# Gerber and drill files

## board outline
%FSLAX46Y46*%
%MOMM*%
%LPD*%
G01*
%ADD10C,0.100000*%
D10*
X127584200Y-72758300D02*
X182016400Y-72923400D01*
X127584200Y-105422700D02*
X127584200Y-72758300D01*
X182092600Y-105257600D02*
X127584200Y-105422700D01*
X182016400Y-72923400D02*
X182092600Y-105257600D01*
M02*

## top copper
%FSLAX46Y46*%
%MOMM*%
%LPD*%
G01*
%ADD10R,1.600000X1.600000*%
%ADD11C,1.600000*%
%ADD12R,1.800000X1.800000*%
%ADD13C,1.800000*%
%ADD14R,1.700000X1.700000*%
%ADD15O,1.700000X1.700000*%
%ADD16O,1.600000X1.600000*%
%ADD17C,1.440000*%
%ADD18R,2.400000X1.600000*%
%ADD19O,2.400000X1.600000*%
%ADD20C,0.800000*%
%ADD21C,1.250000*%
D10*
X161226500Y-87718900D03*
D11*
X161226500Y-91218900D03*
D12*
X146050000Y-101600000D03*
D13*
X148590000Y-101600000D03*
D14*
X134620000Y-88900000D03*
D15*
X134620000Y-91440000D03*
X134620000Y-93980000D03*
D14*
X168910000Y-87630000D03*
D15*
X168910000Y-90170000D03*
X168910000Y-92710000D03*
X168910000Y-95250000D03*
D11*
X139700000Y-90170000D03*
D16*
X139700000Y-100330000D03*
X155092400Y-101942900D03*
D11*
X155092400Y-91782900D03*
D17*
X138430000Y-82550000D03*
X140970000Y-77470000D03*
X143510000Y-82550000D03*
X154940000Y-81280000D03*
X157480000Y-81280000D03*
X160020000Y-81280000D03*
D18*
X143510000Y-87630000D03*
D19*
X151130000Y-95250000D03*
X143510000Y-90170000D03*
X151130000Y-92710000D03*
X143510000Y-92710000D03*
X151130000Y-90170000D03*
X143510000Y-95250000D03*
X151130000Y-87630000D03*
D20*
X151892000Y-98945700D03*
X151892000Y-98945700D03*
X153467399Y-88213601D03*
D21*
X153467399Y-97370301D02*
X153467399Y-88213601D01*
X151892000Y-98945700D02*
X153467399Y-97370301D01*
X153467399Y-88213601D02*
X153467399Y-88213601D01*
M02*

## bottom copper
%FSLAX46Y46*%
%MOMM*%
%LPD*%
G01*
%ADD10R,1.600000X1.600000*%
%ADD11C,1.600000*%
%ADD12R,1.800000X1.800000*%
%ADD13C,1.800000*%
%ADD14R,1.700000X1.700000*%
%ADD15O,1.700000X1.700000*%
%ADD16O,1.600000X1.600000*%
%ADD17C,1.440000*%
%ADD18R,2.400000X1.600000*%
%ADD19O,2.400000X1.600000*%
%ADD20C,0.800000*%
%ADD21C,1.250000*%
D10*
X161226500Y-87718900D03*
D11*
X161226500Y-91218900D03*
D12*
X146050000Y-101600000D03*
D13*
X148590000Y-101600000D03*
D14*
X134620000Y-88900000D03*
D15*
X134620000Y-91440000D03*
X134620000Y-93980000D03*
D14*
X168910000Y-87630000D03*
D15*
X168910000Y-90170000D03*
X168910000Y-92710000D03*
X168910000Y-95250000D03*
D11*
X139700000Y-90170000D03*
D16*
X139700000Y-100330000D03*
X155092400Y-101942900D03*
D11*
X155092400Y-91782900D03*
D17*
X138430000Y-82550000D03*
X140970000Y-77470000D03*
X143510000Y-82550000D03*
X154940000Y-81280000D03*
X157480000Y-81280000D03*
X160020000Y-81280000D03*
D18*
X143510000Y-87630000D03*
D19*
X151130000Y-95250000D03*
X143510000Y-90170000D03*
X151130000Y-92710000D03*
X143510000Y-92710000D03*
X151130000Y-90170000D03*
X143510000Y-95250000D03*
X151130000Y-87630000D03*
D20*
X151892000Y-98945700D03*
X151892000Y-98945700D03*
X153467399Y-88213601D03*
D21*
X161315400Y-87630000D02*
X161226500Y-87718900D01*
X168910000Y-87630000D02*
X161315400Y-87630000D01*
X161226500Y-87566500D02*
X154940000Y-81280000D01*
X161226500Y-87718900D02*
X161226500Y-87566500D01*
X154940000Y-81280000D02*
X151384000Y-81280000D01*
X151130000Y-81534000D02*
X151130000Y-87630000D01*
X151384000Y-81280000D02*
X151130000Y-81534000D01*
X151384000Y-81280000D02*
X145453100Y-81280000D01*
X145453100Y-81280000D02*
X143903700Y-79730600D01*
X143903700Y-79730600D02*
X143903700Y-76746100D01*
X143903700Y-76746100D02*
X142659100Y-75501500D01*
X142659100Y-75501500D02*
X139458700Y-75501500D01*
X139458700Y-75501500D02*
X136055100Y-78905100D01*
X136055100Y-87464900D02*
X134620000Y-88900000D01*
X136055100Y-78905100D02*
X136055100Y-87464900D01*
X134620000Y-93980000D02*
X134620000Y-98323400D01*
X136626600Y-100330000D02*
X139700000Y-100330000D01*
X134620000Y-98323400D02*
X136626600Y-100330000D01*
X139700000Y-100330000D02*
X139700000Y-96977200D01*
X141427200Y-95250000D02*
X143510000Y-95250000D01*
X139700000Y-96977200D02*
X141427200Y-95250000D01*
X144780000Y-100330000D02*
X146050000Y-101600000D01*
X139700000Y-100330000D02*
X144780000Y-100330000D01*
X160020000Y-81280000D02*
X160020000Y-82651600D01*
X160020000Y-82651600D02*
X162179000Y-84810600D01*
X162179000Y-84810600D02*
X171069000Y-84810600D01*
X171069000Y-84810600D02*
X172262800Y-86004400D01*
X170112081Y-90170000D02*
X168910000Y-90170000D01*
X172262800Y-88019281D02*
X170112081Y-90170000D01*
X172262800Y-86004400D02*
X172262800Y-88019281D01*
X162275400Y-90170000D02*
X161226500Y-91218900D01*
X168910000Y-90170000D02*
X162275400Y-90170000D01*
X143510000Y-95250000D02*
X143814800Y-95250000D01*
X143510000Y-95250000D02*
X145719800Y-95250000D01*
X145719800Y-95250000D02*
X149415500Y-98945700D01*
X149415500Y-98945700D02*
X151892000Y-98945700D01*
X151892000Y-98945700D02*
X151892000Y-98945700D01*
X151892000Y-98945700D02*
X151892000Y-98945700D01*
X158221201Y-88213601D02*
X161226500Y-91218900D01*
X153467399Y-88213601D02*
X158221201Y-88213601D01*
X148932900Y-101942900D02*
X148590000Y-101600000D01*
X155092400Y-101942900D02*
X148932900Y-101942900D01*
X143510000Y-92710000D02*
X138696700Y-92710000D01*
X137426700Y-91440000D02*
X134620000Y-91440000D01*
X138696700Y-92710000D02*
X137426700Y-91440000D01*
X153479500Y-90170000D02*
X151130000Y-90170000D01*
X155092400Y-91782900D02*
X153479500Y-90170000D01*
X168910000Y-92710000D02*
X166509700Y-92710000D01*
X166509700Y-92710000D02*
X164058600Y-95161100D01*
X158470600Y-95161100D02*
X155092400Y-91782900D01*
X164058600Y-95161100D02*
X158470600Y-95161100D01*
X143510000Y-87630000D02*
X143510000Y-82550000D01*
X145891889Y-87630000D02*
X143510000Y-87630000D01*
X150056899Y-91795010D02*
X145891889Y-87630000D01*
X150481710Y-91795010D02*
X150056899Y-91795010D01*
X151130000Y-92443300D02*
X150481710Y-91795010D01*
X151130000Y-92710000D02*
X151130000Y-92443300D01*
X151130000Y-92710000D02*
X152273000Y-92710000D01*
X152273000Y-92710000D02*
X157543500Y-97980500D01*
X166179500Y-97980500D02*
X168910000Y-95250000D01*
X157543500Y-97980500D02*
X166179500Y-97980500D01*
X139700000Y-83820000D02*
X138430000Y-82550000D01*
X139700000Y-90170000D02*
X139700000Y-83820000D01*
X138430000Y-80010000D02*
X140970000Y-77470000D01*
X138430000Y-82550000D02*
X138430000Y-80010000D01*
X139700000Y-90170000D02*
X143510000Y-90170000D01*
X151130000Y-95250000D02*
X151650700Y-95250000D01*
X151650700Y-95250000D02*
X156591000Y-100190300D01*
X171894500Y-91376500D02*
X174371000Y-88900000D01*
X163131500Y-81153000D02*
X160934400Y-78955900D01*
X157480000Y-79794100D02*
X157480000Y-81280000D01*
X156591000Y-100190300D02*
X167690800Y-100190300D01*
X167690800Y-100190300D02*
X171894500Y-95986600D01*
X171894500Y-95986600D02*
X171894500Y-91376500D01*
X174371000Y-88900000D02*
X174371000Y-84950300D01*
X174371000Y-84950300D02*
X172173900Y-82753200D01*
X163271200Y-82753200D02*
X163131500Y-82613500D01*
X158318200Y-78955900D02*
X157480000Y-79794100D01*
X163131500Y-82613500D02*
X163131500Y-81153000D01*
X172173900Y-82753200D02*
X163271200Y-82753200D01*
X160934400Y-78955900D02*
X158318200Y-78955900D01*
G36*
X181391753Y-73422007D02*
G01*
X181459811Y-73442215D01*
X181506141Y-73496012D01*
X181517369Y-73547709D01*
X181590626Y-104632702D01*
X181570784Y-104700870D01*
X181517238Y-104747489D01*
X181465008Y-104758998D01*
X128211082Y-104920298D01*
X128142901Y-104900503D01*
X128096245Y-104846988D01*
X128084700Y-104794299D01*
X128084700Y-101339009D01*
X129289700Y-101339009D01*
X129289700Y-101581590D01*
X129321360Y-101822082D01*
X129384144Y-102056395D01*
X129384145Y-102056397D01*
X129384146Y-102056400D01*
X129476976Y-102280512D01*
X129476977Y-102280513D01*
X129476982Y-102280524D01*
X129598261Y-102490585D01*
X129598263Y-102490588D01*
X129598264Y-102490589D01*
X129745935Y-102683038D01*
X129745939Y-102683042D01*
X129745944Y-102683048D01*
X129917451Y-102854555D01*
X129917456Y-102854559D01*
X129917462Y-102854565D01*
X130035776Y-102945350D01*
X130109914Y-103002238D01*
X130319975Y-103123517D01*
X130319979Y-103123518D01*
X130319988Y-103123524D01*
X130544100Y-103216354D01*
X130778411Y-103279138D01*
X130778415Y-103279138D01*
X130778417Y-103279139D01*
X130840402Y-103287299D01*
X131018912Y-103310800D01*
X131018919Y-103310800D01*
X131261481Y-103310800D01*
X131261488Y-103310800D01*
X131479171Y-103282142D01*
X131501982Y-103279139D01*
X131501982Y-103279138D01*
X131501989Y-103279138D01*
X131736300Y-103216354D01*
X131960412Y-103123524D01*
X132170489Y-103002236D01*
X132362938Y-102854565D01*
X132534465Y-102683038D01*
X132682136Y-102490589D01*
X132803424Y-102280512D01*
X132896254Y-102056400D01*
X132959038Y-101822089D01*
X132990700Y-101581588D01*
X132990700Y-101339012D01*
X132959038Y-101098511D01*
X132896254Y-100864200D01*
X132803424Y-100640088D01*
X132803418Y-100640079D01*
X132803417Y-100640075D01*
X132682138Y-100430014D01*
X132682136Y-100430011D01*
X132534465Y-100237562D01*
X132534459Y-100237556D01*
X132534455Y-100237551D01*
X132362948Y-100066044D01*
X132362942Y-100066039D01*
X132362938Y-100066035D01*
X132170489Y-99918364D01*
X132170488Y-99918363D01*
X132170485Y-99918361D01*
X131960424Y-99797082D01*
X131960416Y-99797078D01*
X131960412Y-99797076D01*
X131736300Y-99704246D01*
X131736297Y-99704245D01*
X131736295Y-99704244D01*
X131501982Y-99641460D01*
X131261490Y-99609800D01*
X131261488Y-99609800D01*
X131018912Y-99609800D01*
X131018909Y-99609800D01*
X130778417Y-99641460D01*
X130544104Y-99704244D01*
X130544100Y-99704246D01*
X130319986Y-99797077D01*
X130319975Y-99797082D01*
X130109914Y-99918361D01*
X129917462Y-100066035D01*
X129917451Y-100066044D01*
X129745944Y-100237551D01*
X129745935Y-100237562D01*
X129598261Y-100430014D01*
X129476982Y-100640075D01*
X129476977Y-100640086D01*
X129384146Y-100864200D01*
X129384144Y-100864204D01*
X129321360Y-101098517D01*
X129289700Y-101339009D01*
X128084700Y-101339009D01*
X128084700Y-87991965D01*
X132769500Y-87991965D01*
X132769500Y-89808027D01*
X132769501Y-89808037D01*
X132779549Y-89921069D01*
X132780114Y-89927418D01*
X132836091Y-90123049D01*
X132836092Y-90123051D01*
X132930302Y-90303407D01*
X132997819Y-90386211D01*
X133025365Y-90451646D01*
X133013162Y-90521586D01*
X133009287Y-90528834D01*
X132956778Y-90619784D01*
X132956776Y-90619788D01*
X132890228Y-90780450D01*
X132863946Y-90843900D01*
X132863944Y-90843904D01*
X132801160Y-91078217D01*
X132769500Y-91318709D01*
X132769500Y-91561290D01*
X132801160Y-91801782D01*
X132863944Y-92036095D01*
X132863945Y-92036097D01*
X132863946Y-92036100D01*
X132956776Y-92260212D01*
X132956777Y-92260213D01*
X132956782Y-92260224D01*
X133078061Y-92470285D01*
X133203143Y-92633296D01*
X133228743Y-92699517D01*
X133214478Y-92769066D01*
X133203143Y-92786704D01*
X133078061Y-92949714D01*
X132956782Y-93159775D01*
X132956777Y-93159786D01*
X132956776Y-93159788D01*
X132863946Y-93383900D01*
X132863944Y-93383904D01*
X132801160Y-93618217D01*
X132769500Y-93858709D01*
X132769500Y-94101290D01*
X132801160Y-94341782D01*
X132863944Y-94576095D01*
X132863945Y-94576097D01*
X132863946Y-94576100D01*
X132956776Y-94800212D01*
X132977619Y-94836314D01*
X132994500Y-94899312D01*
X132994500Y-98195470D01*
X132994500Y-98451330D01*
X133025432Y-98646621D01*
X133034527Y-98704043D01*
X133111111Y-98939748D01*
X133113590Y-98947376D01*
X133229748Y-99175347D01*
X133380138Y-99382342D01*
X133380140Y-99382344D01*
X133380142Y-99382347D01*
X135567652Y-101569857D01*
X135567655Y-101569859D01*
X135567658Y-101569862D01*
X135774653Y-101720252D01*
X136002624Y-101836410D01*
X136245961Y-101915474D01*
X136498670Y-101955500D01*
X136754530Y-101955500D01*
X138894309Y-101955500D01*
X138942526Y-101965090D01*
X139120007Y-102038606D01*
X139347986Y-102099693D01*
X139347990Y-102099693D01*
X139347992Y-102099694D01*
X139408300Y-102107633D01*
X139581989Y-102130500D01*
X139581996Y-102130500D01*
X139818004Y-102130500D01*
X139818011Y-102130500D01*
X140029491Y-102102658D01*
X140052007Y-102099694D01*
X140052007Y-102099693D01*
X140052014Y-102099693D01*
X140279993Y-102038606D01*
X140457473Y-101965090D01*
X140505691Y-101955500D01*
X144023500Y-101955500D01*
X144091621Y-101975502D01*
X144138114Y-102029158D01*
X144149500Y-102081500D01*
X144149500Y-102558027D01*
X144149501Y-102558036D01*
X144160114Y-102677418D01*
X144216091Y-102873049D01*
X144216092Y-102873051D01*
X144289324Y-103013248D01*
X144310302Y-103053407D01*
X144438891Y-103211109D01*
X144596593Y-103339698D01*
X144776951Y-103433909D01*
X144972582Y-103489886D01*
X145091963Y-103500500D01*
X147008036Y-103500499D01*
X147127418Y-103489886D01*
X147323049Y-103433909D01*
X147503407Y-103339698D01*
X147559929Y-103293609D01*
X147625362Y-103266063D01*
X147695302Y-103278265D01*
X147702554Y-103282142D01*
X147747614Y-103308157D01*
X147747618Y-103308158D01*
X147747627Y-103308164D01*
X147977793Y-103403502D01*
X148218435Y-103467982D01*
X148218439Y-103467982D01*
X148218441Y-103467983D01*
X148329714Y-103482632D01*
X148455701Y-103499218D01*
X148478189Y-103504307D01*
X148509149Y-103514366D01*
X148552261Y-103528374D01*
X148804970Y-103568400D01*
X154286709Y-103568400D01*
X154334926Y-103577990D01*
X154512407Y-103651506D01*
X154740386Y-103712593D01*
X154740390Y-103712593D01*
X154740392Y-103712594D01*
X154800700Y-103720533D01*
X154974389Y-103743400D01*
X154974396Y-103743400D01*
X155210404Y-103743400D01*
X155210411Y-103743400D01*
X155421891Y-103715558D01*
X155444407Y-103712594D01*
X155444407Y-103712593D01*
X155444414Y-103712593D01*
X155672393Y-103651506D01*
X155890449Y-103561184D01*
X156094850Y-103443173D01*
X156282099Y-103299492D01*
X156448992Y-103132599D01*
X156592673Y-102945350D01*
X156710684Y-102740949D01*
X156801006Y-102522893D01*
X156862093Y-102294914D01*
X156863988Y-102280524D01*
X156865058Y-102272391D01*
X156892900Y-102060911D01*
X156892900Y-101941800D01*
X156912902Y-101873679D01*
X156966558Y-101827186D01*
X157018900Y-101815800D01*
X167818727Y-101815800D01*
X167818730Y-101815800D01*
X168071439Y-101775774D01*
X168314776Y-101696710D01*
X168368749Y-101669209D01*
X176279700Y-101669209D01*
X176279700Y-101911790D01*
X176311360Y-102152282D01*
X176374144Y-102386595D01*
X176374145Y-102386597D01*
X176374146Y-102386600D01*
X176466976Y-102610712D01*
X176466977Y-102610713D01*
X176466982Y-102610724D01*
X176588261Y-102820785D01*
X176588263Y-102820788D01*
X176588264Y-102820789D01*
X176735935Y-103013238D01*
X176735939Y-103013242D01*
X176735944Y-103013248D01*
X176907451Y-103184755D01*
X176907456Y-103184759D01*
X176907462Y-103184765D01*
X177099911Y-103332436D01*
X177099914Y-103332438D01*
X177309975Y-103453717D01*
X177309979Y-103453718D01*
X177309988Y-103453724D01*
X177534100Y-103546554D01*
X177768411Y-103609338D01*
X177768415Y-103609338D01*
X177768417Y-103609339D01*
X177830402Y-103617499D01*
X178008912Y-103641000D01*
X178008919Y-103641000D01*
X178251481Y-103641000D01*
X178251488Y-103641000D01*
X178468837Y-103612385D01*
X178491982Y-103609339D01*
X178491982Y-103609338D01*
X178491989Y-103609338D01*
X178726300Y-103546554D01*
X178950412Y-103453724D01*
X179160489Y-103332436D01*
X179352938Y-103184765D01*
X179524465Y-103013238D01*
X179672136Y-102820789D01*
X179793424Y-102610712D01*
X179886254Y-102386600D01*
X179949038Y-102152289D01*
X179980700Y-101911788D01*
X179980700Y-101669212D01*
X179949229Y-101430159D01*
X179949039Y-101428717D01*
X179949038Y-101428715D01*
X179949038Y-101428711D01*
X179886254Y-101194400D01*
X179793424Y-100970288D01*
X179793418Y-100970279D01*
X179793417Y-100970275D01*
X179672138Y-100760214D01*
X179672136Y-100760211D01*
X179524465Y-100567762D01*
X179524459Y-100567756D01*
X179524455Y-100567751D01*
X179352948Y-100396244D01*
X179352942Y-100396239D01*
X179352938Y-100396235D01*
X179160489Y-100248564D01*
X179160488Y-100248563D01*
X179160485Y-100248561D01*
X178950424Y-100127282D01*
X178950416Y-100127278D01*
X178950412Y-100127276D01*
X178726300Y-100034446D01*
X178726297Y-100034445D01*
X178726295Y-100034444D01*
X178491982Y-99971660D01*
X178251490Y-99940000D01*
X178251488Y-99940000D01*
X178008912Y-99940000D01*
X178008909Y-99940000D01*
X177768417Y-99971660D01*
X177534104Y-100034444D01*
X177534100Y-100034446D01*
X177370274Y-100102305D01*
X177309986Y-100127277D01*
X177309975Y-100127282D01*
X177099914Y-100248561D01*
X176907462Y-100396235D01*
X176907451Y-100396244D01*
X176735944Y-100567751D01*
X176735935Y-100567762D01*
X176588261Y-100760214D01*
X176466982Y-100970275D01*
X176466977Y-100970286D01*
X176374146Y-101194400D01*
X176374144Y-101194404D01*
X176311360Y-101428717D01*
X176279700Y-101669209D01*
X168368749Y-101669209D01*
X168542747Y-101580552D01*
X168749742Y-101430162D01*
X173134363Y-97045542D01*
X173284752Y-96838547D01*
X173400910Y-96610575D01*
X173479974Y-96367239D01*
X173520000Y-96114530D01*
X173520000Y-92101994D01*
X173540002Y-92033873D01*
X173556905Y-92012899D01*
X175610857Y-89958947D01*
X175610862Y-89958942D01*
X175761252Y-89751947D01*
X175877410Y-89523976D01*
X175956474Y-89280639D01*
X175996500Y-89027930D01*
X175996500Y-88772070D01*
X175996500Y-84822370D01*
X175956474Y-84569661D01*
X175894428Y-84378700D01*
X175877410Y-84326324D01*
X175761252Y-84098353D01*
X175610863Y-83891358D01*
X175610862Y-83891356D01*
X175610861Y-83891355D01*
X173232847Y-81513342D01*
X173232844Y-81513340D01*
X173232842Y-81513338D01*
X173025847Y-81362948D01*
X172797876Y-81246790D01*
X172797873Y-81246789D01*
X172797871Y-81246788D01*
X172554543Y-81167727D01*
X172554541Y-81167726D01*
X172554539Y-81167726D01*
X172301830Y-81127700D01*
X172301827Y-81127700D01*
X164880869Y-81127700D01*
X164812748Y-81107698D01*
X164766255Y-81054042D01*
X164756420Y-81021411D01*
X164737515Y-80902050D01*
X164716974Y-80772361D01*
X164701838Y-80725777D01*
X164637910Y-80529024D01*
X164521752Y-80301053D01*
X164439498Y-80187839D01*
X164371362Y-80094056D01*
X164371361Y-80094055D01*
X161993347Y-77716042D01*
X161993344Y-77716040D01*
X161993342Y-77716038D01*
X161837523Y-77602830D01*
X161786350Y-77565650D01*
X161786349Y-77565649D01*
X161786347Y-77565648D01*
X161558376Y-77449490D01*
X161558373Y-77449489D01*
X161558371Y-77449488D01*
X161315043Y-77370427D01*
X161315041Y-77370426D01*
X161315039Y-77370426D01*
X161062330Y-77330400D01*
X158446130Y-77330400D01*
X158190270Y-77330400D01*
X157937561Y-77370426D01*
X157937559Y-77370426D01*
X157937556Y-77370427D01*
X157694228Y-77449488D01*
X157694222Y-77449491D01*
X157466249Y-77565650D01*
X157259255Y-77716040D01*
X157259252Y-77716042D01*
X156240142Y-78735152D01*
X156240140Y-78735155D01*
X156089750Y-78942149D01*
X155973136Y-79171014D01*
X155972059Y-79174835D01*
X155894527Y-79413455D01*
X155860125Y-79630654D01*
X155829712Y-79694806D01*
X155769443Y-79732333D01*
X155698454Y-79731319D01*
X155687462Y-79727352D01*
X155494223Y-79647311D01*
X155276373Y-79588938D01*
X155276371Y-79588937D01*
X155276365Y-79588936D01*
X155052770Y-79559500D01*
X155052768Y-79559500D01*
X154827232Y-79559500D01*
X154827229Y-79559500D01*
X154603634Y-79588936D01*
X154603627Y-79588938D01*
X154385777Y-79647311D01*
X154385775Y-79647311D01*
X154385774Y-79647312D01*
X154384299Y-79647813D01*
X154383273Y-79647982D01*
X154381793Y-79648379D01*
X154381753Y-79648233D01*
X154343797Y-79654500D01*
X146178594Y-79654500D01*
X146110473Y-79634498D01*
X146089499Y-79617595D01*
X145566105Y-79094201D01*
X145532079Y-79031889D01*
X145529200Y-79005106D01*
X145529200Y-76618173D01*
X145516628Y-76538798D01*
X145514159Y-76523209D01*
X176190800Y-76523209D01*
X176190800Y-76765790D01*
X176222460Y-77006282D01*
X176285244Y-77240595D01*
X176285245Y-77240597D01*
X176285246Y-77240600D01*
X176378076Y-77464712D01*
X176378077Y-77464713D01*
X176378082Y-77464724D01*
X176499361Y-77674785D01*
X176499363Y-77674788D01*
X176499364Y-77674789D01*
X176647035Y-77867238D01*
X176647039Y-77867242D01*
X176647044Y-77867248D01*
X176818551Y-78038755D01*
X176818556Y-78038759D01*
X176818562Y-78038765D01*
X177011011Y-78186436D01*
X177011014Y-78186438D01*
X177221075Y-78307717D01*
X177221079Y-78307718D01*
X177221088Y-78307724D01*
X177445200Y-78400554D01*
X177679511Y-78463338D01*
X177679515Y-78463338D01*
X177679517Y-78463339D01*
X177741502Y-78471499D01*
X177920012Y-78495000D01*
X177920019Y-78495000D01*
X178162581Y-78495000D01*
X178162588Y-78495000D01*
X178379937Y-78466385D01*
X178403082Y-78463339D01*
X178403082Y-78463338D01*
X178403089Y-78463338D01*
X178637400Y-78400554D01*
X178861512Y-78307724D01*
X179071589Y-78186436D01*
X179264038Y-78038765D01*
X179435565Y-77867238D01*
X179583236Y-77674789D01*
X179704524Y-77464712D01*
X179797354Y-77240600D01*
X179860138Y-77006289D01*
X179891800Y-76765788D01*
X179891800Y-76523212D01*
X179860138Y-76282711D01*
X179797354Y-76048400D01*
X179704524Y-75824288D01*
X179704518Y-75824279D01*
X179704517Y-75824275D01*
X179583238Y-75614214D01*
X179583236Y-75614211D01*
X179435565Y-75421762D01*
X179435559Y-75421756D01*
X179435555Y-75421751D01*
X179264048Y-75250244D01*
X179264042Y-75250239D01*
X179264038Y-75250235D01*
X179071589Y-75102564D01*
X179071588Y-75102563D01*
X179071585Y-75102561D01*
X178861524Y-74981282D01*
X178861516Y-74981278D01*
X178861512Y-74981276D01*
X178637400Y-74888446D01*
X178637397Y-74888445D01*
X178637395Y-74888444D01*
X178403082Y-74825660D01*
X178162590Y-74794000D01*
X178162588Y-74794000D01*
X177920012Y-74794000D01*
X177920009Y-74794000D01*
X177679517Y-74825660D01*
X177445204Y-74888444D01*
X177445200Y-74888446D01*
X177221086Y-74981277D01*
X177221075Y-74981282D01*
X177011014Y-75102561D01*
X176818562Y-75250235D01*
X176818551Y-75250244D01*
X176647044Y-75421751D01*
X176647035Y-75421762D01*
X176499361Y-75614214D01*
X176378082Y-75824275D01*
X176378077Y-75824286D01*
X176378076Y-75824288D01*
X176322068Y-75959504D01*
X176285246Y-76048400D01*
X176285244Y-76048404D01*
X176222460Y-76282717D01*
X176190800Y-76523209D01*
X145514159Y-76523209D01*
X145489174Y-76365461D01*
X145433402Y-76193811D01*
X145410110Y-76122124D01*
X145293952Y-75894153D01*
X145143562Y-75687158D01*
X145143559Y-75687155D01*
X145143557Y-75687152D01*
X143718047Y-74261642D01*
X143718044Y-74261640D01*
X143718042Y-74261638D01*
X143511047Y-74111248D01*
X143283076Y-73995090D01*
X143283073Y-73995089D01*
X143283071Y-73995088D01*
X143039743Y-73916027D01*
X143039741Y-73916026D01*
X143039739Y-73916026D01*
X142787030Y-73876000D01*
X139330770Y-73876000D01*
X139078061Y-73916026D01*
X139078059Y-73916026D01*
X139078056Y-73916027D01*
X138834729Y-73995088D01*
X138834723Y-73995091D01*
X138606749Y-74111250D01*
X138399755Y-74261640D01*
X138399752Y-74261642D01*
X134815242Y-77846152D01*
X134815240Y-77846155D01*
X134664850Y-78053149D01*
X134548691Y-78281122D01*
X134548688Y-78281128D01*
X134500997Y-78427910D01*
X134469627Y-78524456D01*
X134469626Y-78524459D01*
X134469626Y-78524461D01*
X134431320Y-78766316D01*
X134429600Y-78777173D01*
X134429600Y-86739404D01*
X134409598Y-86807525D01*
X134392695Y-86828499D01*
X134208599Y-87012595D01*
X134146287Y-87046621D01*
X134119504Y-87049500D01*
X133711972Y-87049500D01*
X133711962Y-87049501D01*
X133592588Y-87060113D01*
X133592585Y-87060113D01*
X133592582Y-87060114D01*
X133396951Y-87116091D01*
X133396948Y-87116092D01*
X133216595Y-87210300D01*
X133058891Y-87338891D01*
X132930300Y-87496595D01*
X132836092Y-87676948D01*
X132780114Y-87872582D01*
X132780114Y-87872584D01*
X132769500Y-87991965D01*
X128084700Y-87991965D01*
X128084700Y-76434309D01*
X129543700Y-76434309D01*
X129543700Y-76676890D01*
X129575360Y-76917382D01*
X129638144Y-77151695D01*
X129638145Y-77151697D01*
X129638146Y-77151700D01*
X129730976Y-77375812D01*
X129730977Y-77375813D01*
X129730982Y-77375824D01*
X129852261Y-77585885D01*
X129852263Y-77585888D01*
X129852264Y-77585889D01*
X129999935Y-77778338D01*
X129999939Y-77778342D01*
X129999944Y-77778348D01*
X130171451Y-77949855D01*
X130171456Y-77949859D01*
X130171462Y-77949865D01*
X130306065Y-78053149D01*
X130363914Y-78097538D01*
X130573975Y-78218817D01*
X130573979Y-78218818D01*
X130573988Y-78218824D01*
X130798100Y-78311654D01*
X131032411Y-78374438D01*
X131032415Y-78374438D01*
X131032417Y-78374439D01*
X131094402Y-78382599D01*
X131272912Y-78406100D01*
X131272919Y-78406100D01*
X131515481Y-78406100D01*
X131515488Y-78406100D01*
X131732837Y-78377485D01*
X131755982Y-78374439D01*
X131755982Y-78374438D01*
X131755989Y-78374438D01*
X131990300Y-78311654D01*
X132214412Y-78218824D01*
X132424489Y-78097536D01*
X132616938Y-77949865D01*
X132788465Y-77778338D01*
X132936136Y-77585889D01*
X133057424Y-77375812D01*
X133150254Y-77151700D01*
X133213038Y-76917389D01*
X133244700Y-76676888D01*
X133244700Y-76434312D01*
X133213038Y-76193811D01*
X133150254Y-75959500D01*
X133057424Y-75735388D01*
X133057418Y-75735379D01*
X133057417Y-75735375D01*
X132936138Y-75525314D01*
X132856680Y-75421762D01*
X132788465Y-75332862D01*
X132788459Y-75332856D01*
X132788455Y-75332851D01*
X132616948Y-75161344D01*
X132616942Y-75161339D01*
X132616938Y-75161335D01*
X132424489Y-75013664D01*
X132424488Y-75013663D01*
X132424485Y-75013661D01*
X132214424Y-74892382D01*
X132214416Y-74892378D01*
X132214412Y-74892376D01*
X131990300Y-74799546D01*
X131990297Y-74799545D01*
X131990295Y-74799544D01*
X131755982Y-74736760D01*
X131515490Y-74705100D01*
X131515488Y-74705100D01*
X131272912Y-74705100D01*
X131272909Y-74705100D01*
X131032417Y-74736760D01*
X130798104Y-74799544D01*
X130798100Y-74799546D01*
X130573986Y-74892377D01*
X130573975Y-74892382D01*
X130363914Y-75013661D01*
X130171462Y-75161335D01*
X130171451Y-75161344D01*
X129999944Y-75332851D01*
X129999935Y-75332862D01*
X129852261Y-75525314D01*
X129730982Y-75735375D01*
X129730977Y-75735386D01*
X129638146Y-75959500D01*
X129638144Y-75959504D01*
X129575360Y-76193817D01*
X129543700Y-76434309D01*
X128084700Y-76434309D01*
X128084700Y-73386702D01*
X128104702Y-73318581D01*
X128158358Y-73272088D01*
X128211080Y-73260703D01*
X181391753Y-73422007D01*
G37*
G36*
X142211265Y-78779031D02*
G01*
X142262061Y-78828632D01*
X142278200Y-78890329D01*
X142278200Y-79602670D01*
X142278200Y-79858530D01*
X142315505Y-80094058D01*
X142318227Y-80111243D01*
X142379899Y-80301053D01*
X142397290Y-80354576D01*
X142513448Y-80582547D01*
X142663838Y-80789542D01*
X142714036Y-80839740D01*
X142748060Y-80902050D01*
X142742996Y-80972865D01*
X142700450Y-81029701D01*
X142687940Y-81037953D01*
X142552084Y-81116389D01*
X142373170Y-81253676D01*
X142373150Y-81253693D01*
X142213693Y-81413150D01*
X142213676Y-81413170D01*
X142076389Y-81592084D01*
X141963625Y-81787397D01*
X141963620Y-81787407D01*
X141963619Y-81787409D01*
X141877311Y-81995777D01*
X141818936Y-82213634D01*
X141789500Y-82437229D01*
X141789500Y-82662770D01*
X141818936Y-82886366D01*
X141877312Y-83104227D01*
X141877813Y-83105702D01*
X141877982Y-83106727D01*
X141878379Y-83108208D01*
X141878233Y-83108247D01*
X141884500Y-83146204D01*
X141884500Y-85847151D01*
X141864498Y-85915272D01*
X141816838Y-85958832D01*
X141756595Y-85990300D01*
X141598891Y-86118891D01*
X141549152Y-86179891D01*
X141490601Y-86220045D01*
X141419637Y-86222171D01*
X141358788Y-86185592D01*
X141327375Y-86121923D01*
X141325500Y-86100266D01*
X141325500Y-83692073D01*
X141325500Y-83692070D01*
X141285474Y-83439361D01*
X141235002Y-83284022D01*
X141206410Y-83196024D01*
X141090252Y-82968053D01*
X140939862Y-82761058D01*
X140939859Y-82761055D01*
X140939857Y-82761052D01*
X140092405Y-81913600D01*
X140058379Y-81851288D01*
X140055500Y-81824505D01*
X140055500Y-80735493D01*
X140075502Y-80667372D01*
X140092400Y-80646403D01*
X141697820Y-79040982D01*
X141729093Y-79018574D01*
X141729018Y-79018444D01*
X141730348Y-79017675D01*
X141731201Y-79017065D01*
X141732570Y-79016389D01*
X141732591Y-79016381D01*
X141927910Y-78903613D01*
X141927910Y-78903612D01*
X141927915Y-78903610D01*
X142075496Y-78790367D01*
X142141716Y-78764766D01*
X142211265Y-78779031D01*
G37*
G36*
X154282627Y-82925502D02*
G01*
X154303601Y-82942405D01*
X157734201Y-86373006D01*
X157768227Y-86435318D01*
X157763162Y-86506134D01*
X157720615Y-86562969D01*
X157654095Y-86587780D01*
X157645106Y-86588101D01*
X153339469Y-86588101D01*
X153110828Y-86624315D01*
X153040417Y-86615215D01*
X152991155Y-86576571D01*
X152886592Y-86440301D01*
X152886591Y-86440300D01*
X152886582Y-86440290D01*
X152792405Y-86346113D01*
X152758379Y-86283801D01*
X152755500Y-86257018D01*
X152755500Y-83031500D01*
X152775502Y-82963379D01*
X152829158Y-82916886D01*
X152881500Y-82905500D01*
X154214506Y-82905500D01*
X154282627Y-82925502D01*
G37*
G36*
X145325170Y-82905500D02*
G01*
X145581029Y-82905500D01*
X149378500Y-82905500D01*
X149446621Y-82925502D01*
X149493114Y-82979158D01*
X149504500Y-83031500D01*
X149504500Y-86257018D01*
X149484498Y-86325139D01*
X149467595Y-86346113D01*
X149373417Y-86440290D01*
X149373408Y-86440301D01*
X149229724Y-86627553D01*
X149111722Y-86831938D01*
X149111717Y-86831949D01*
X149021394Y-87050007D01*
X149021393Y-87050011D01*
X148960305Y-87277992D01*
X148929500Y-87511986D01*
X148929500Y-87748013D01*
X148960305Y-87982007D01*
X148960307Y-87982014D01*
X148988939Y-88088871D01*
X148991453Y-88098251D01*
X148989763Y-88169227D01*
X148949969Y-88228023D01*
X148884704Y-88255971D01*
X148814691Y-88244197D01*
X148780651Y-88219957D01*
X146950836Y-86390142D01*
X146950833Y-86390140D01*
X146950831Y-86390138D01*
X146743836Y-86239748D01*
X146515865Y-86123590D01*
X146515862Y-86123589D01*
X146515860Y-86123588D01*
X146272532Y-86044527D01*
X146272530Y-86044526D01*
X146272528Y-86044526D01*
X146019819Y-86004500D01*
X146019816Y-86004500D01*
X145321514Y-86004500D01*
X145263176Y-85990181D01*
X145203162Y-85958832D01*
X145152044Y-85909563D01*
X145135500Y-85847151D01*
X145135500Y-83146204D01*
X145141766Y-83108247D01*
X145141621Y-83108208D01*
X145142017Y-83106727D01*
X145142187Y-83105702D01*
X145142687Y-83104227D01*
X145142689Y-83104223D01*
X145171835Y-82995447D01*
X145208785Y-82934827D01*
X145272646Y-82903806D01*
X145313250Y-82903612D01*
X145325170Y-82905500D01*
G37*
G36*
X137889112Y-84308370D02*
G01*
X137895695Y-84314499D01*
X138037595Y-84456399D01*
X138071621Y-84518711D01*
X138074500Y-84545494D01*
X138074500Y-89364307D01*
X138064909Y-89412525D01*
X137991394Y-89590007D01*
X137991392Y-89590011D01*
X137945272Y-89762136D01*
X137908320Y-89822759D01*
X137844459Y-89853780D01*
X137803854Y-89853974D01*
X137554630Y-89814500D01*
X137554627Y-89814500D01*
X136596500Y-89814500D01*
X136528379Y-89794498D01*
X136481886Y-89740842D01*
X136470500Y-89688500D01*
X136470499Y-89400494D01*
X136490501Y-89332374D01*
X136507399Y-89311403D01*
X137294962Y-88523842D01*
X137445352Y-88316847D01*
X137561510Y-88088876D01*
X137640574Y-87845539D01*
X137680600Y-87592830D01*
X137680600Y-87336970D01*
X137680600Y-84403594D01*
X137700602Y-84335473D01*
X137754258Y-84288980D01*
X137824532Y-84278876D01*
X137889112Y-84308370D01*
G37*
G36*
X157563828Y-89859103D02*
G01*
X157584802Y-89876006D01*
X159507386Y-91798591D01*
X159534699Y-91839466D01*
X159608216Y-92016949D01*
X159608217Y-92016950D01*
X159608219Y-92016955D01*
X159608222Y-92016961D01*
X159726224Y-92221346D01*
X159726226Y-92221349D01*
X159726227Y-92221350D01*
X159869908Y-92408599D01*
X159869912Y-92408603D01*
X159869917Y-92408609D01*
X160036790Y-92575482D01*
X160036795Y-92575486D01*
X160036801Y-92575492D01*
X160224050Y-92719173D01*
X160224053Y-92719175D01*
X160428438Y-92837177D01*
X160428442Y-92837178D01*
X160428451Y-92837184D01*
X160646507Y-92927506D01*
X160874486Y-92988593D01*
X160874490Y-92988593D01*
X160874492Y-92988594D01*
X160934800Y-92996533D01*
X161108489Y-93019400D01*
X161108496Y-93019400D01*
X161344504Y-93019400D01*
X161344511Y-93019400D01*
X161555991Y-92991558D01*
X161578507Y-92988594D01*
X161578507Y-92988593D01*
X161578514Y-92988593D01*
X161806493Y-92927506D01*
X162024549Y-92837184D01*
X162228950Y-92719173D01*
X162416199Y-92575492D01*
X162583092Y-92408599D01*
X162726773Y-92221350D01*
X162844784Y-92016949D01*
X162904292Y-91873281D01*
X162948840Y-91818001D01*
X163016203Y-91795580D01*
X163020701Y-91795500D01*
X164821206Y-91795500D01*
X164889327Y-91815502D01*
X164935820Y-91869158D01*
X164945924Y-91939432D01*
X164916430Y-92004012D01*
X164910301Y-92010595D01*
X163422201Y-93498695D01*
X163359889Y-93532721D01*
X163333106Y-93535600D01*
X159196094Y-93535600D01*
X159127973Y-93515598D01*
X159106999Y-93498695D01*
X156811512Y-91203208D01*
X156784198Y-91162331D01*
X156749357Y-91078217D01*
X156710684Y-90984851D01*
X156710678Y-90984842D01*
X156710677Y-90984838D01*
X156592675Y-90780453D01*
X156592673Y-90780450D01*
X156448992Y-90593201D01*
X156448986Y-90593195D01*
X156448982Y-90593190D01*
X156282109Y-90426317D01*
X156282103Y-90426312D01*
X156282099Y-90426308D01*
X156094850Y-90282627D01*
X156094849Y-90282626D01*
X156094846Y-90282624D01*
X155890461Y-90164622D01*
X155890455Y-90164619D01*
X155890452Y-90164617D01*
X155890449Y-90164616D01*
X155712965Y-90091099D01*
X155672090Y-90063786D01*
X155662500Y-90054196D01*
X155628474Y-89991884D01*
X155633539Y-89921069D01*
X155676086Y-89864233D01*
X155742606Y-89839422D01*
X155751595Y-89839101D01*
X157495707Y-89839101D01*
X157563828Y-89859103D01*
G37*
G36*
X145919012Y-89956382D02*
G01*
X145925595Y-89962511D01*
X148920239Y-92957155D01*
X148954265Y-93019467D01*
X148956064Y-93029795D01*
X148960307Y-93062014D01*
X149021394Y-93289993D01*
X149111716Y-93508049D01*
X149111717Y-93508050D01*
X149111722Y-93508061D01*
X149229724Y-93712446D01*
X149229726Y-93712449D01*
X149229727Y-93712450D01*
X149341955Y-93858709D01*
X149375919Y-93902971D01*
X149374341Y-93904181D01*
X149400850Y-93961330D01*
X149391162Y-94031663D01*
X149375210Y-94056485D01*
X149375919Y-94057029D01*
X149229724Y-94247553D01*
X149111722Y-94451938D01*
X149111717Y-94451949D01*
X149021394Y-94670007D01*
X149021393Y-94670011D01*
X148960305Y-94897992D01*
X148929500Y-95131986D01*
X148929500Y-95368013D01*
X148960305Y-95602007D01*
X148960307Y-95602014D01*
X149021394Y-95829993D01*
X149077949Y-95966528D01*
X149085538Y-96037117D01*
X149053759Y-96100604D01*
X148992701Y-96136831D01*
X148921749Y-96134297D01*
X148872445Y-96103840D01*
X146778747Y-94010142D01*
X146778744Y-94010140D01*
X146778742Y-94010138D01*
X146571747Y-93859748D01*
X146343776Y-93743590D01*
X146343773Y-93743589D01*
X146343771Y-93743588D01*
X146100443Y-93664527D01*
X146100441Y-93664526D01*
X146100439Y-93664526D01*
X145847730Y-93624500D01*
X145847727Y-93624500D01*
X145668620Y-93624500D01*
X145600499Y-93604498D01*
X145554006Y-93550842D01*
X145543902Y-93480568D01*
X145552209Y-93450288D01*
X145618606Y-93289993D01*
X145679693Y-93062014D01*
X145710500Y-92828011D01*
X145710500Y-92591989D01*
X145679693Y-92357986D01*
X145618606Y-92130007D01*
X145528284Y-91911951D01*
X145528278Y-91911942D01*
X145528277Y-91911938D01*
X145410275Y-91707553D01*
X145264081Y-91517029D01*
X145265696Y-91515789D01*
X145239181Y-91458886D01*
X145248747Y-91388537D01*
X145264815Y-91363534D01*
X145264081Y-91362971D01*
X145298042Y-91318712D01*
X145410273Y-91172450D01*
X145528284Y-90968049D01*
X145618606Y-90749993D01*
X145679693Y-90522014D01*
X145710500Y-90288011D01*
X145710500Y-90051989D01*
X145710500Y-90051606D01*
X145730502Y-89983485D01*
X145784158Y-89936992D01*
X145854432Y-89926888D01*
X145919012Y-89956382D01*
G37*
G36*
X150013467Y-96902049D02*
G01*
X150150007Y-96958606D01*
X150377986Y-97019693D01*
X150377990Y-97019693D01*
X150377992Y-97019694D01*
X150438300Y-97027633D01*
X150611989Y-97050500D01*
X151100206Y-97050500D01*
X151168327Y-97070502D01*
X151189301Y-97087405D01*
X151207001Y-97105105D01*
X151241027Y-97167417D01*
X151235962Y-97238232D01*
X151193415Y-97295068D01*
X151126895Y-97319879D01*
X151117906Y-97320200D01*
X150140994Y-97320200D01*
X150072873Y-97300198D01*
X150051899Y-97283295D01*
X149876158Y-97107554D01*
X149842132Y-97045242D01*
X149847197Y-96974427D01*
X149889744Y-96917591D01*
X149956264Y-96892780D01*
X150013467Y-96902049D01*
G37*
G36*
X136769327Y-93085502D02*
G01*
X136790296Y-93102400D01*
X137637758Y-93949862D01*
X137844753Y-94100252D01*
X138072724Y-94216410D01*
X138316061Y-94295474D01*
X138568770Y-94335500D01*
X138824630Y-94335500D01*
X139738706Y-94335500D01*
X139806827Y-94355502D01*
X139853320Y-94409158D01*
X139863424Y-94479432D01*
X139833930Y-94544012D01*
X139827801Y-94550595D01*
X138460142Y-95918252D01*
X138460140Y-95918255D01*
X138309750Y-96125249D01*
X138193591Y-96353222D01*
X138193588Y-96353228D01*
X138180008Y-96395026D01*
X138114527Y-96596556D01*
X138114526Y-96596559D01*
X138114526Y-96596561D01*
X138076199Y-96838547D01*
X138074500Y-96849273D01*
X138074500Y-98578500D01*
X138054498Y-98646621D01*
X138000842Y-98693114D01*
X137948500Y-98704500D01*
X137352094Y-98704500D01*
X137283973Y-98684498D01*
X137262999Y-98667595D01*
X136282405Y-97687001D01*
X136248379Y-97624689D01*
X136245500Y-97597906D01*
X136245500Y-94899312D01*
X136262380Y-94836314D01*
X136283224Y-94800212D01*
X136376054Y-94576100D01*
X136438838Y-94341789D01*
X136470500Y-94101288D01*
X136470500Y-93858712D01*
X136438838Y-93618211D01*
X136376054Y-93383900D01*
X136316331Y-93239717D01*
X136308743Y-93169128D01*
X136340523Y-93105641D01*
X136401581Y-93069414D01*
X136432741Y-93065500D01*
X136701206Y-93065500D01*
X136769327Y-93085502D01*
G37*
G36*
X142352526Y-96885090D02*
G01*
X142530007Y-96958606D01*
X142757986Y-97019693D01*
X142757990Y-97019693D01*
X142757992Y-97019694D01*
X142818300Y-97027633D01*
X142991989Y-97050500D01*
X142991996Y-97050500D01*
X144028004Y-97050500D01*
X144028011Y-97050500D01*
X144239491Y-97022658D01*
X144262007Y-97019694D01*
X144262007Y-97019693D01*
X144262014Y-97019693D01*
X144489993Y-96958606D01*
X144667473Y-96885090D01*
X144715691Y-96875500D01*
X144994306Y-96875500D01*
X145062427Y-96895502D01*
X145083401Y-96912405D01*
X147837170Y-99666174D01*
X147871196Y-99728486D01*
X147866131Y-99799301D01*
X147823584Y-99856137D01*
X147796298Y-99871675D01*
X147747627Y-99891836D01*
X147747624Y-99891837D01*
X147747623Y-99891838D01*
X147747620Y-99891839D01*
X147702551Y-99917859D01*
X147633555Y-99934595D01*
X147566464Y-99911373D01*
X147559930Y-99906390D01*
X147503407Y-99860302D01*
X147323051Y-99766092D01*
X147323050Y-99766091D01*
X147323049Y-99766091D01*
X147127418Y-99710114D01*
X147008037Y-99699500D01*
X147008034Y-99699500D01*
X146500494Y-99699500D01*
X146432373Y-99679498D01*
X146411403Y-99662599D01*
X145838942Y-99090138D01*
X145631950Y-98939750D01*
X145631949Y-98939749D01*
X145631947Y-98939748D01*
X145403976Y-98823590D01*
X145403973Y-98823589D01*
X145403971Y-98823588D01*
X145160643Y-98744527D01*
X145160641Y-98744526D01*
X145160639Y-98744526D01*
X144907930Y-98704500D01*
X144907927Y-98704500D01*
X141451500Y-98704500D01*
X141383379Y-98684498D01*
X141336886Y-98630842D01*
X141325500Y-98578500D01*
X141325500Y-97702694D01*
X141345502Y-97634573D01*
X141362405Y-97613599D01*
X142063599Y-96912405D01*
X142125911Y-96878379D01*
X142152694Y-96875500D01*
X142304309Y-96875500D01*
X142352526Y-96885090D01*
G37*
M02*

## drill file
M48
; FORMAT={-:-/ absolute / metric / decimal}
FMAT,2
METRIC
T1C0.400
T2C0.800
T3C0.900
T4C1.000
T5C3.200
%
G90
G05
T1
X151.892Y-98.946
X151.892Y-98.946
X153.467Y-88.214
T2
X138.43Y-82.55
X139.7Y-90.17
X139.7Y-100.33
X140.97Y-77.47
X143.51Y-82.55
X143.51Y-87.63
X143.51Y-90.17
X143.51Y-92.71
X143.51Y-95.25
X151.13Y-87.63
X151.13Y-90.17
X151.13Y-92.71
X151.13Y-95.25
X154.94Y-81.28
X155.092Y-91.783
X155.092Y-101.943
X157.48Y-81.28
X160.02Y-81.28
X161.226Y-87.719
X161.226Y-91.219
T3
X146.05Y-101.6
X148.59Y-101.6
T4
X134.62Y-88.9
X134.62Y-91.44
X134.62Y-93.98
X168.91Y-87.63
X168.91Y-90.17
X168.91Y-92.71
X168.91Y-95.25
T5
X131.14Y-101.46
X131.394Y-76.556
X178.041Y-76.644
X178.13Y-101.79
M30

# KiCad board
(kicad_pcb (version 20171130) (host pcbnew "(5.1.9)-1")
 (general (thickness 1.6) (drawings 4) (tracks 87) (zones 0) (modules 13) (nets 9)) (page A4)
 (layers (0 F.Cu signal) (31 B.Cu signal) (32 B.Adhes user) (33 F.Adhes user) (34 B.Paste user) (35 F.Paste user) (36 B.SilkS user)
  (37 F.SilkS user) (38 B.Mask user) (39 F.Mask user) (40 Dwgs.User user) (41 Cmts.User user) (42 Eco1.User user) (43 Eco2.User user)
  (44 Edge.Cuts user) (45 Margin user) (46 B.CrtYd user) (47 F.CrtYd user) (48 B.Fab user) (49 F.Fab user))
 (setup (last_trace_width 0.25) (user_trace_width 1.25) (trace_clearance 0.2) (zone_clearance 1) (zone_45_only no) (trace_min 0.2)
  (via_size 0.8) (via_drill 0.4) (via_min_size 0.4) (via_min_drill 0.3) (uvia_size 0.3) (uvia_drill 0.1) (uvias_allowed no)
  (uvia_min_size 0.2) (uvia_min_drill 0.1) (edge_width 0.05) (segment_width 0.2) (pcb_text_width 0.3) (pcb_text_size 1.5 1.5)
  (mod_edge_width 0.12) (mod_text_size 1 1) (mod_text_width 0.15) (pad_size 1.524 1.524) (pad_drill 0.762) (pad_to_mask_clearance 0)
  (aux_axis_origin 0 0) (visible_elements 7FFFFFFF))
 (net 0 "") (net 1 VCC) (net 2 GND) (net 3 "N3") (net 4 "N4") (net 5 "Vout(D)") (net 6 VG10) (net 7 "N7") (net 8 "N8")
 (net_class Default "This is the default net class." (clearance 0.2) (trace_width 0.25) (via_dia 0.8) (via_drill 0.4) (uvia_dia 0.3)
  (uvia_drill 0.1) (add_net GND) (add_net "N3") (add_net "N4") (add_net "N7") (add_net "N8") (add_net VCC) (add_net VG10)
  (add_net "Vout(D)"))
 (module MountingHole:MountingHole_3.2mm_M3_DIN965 (layer F.Cu) (at 131.3942 76.5556)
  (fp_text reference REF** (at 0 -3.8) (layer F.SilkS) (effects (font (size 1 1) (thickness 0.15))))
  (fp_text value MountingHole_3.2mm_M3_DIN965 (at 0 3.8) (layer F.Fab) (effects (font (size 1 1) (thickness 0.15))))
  (pad 1 np_thru_hole circle (at 0 0) (size 3.2 3.2) (drill 3.2) (layers *.Cu *.Mask)))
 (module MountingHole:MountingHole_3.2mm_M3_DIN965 (layer F.Cu) (at 131.1402 101.4603)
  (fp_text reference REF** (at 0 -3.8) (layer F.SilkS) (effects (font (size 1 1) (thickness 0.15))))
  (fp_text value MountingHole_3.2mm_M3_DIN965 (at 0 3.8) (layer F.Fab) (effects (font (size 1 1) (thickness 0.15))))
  (pad 1 np_thru_hole circle (at 0 0) (size 3.2 3.2) (drill 3.2) (layers *.Cu *.Mask)))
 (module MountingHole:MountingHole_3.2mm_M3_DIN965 (layer F.Cu) (at 178.1302 101.7905)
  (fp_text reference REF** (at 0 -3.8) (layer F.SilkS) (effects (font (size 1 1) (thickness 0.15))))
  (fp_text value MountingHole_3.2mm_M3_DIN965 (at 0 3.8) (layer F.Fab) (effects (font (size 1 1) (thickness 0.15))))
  (pad 1 np_thru_hole circle (at 0 0) (size 3.2 3.2) (drill 3.2) (layers *.Cu *.Mask)))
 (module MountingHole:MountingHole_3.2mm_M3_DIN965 (layer F.Cu) (at 178.0413 76.6445)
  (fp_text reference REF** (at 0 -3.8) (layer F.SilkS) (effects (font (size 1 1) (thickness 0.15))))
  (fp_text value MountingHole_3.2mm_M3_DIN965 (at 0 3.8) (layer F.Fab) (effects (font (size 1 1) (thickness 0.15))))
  (pad 1 np_thru_hole circle (at 0 0) (size 3.2 3.2) (drill 3.2) (layers *.Cu *.Mask)))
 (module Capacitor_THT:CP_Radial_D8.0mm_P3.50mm (layer F.Cu) (at 161.2265 87.7189 270)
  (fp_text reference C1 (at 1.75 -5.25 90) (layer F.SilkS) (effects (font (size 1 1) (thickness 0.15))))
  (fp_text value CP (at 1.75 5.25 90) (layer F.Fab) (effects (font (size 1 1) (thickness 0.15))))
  (pad 1 thru_hole rect (at 0 0 270) (size 1.6 1.6) (drill 0.8) (layers *.Cu *.Mask) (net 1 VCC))
  (pad 2 thru_hole circle (at 3.5 0 270) (size 1.6 1.6) (drill 0.8) (layers *.Cu *.Mask) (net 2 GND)))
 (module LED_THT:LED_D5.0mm (layer F.Cu) (at 146.05 101.6)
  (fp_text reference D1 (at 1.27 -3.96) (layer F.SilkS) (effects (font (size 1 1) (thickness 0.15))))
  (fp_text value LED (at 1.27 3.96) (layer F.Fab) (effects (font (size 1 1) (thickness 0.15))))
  (pad 1 thru_hole rect (at 0 0) (size 1.8 1.8) (drill 0.9) (layers *.Cu *.Mask) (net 2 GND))
  (pad 2 thru_hole circle (at 2.54 0) (size 1.8 1.8) (drill 0.9) (layers *.Cu *.Mask) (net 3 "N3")))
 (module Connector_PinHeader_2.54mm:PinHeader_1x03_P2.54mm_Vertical (layer F.Cu) (at 134.62 88.9)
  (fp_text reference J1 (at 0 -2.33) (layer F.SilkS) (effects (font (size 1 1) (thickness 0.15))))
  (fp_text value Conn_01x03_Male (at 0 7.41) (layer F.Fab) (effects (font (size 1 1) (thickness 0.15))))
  (pad 1 thru_hole rect (at 0 0) (size 1.7 1.7) (drill 1) (layers *.Cu *.Mask) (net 1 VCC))
  (pad 2 thru_hole oval (at 0 2.54) (size 1.7 1.7) (drill 1) (layers *.Cu *.Mask) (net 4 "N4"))
  (pad 3 thru_hole oval (at 0 5.08) (size 1.7 1.7) (drill 1) (layers *.Cu *.Mask) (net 2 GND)))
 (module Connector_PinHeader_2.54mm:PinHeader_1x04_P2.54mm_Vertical (layer F.Cu) (at 168.91 87.63)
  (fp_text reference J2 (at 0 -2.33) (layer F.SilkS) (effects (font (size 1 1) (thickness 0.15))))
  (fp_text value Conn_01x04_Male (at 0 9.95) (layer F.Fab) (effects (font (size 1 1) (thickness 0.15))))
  (pad 1 thru_hole rect (at 0 0) (size 1.7 1.7) (drill 1) (layers *.Cu *.Mask) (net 1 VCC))
  (pad 2 thru_hole oval (at 0 2.54) (size 1.7 1.7) (drill 1) (layers *.Cu *.Mask) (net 2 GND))
  (pad 3 thru_hole oval (at 0 5.08) (size 1.7 1.7) (drill 1) (layers *.Cu *.Mask) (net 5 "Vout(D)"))
  (pad 4 thru_hole oval (at 0 7.62) (size 1.7 1.7) (drill 1) (layers *.Cu *.Mask) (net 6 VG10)))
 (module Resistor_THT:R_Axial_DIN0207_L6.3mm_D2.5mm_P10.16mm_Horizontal (layer F.Cu) (at 139.7 90.17 270)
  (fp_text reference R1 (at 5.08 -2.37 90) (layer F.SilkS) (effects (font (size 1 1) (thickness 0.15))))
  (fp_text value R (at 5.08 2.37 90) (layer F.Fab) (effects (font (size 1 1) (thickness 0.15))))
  (pad 1 thru_hole circle (at 0 0 270) (size 1.6 1.6) (drill 0.8) (layers *.Cu *.Mask) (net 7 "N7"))
  (pad 2 thru_hole oval (at 10.16 0 270) (size 1.6 1.6) (drill 0.8) (layers *.Cu *.Mask) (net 2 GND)))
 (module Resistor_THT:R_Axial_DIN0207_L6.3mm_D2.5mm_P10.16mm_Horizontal (layer F.Cu) (at 155.0924 91.7829 270)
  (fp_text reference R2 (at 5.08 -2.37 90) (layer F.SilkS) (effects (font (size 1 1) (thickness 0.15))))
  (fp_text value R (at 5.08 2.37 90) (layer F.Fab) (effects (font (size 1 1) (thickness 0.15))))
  (pad 2 thru_hole oval (at 10.16 0 270) (size 1.6 1.6) (drill 0.8) (layers *.Cu *.Mask) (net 3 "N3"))
  (pad 1 thru_hole circle (at 0 0 270) (size 1.6 1.6) (drill 0.8) (layers *.Cu *.Mask) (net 5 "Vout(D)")))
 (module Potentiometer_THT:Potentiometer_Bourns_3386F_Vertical (layer F.Cu) (at 143.51 82.55 90)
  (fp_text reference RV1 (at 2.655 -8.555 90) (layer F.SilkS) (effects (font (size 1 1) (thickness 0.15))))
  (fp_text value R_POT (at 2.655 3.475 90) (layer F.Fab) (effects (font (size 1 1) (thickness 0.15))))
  (pad 3 thru_hole circle (at 0 -5.08 90) (size 1.44 1.44) (drill 0.8) (layers *.Cu *.Mask) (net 7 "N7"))
  (pad 2 thru_hole circle (at 5.08 -2.54 90) (size 1.44 1.44) (drill 0.8) (layers *.Cu *.Mask) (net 7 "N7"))
  (pad 1 thru_hole circle (at 0 0 90) (size 1.44 1.44) (drill 0.8) (layers *.Cu *.Mask) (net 6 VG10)))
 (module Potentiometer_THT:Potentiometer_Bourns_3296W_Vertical (layer F.Cu) (at 154.94 81.28 180)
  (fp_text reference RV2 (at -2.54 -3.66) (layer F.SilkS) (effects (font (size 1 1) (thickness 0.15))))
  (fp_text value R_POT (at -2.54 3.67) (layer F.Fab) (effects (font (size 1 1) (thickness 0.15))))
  (pad 1 thru_hole circle (at 0 0 180) (size 1.44 1.44) (drill 0.8) (layers *.Cu *.Mask) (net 1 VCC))
  (pad 2 thru_hole circle (at -2.54 0 180) (size 1.44 1.44) (drill 0.8) (layers *.Cu *.Mask) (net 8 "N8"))
  (pad 3 thru_hole circle (at -5.08 0 180) (size 1.44 1.44) (drill 0.8) (layers *.Cu *.Mask) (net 2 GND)))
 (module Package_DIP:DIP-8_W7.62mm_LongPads (layer F.Cu) (at 143.51 87.63)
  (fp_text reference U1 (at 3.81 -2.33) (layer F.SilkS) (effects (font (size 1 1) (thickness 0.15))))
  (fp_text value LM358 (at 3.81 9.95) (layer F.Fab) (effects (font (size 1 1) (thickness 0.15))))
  (pad 1 thru_hole rect (at 0 0) (size 2.4 1.6) (drill 0.8) (layers *.Cu *.Mask) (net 6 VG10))
  (pad 5 thru_hole oval (at 7.62 7.62) (size 2.4 1.6) (drill 0.8) (layers *.Cu *.Mask) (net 8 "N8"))
  (pad 2 thru_hole oval (at 0 2.54) (size 2.4 1.6) (drill 0.8) (layers *.Cu *.Mask) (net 7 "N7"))
  (pad 6 thru_hole oval (at 7.62 5.08) (size 2.4 1.6) (drill 0.8) (layers *.Cu *.Mask) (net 6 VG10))
  (pad 3 thru_hole oval (at 0 5.08) (size 2.4 1.6) (drill 0.8) (layers *.Cu *.Mask) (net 4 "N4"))
  (pad 7 thru_hole oval (at 7.62 2.54) (size 2.4 1.6) (drill 0.8) (layers *.Cu *.Mask) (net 5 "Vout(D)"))
  (pad 4 thru_hole oval (at 0 7.62) (size 2.4 1.6) (drill 0.8) (layers *.Cu *.Mask) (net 2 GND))
  (pad 8 thru_hole oval (at 7.62 0) (size 2.4 1.6) (drill 0.8) (layers *.Cu *.Mask) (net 1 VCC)))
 (gr_line (start 127.5842 72.7583) (end 182.0164 72.9234) (layer Edge.Cuts) (width 0.1))
 (gr_line (start 127.5842 105.4227) (end 127.5842 72.7583) (layer Edge.Cuts) (width 0.1))
 (gr_line (start 182.0926 105.2576) (end 127.5842 105.4227) (layer Edge.Cuts) (width 0.1))
 (gr_line (start 182.0164 72.9234) (end 182.0926 105.2576) (layer Edge.Cuts) (width 0.1))
 (segment (start 161.3154 87.63) (end 161.2265 87.7189) (width 1.25) (layer B.Cu) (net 1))
 (segment (start 168.91 87.63) (end 161.3154 87.63) (width 1.25) (layer B.Cu) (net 1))
 (segment (start 161.2265 87.5665) (end 154.94 81.28) (width 1.25) (layer B.Cu) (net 1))
 (segment (start 161.2265 87.7189) (end 161.2265 87.5665) (width 1.25) (layer B.Cu) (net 1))
 (segment (start 154.94 81.28) (end 151.384 81.28) (width 1.25) (layer B.Cu) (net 1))
 (segment (start 151.13 81.534) (end 151.13 87.63) (width 1.25) (layer B.Cu) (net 1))
 (segment (start 151.384 81.28) (end 151.13 81.534) (width 1.25) (layer B.Cu) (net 1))
 (segment (start 151.384 81.28) (end 145.4531 81.28) (width 1.25) (layer B.Cu) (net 1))
 (segment (start 145.4531 81.28) (end 143.9037 79.7306) (width 1.25) (layer B.Cu) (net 1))
 (segment (start 143.9037 79.7306) (end 143.9037 76.7461) (width 1.25) (layer B.Cu) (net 1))
 (segment (start 143.9037 76.7461) (end 142.6591 75.5015) (width 1.25) (layer B.Cu) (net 1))
 (segment (start 142.6591 75.5015) (end 139.4587 75.5015) (width 1.25) (layer B.Cu) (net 1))
 (segment (start 139.4587 75.5015) (end 136.0551 78.9051) (width 1.25) (layer B.Cu) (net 1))
 (segment (start 136.0551 87.4649) (end 134.62 88.9) (width 1.25) (layer B.Cu) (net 1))
 (segment (start 136.0551 78.9051) (end 136.0551 87.4649) (width 1.25) (layer B.Cu) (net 1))
 (segment (start 134.62 93.98) (end 134.62 98.3234) (width 1.25) (layer B.Cu) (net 2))
 (segment (start 136.6266 100.33) (end 139.7 100.33) (width 1.25) (layer B.Cu) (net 2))
 (segment (start 134.62 98.3234) (end 136.6266 100.33) (width 1.25) (layer B.Cu) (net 2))
 (segment (start 139.7 100.33) (end 139.7 96.9772) (width 1.25) (layer B.Cu) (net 2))
 (segment (start 141.4272 95.25) (end 143.51 95.25) (width 1.25) (layer B.Cu) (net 2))
 (segment (start 139.7 96.9772) (end 141.4272 95.25) (width 1.25) (layer B.Cu) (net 2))
 (segment (start 144.78 100.33) (end 146.05 101.6) (width 1.25) (layer B.Cu) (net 2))
 (segment (start 139.7 100.33) (end 144.78 100.33) (width 1.25) (layer B.Cu) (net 2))
 (segment (start 160.02 81.28) (end 160.02 82.6516) (width 1.25) (layer B.Cu) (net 2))
 (segment (start 160.02 82.6516) (end 162.179 84.8106) (width 1.25) (layer B.Cu) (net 2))
 (segment (start 162.179 84.8106) (end 171.069 84.8106) (width 1.25) (layer B.Cu) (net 2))
 (segment (start 171.069 84.8106) (end 172.2628 86.0044) (width 1.25) (layer B.Cu) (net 2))
 (segment (start 170.112081 90.17) (end 168.91 90.17) (width 1.25) (layer B.Cu) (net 2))
 (segment (start 172.2628 88.019281) (end 170.112081 90.17) (width 1.25) (layer B.Cu) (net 2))
 (segment (start 172.2628 86.0044) (end 172.2628 88.019281) (width 1.25) (layer B.Cu) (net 2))
 (segment (start 162.2754 90.17) (end 161.2265 91.2189) (width 1.25) (layer B.Cu) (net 2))
 (segment (start 168.91 90.17) (end 162.2754 90.17) (width 1.25) (layer B.Cu) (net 2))
 (segment (start 143.51 95.25) (end 143.8148 95.25) (width 1.25) (layer B.Cu) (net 2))
 (segment (start 143.51 95.25) (end 145.7198 95.25) (width 1.25) (layer B.Cu) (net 2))
 (segment (start 145.7198 95.25) (end 149.4155 98.9457) (width 1.25) (layer B.Cu) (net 2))
 (segment (start 149.4155 98.9457) (end 151.892 98.9457) (width 1.25) (layer B.Cu) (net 2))
 (segment (start 151.892 98.9457) (end 151.892 98.9457) (width 1.25) (layer B.Cu) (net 2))
 (via (at 151.892 98.9457) (size 0.8) (drill 0.4) (layers F.Cu B.Cu) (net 2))
 (segment (start 151.892 98.9457) (end 151.892 98.9457) (width 1.25) (layer B.Cu) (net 2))
 (via (at 151.892 98.9457) (size 0.8) (drill 0.4) (layers F.Cu B.Cu) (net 2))
 (segment (start 153.467399 97.370301) (end 153.467399 88.213601) (width 1.25) (layer F.Cu) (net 2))
 (segment (start 151.892 98.9457) (end 153.467399 97.370301) (width 1.25) (layer F.Cu) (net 2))
 (segment (start 153.467399 88.213601) (end 153.467399 88.213601) (width 1.25) (layer F.Cu) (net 2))
 (via (at 153.467399 88.213601) (size 0.8) (drill 0.4) (layers F.Cu B.Cu) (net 2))
 (segment (start 158.221201 88.213601) (end 161.2265 91.2189) (width 1.25) (layer B.Cu) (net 2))
 (segment (start 153.467399 88.213601) (end 158.221201 88.213601) (width 1.25) (layer B.Cu) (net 2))
 (segment (start 148.9329 101.9429) (end 148.59 101.6) (width 1.25) (layer B.Cu) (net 3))
 (segment (start 155.0924 101.9429) (end 148.9329 101.9429) (width 1.25) (layer B.Cu) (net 3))
 (segment (start 143.51 92.71) (end 138.6967 92.71) (width 1.25) (layer B.Cu) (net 4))
 (segment (start 137.4267 91.44) (end 134.62 91.44) (width 1.25) (layer B.Cu) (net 4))
 (segment (start 138.6967 92.71) (end 137.4267 91.44) (width 1.25) (layer B.Cu) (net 4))
 (segment (start 153.4795 90.17) (end 151.13 90.17) (width 1.25) (layer B.Cu) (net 5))
 (segment (start 155.0924 91.7829) (end 153.4795 90.17) (width 1.25) (layer B.Cu) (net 5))
 (segment (start 168.91 92.71) (end 166.5097 92.71) (width 1.25) (layer B.Cu) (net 5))
 (segment (start 166.5097 92.71) (end 164.0586 95.1611) (width 1.25) (layer B.Cu) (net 5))
 (segment (start 158.4706 95.1611) (end 155.0924 91.7829) (width 1.25) (layer B.Cu) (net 5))
 (segment (start 164.0586 95.1611) (end 158.4706 95.1611) (width 1.25) (layer B.Cu) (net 5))
 (segment (start 143.51 87.63) (end 143.51 82.55) (width 1.25) (layer B.Cu) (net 6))
 (segment (start 145.891889 87.63) (end 143.51 87.63) (width 1.25) (layer B.Cu) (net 6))
 (segment (start 150.056899 91.79501) (end 145.891889 87.63) (width 1.25) (layer B.Cu) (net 6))
 (segment (start 150.48171 91.79501) (end 150.056899 91.79501) (width 1.25) (layer B.Cu) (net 6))
 (segment (start 151.13 92.4433) (end 150.48171 91.79501) (width 1.25) (layer B.Cu) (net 6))
 (segment (start 151.13 92.71) (end 151.13 92.4433) (width 1.25) (layer B.Cu) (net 6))
 (segment (start 151.13 92.71) (end 152.273 92.71) (width 1.25) (layer B.Cu) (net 6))
 (segment (start 152.273 92.71) (end 157.5435 97.9805) (width 1.25) (layer B.Cu) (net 6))
 (segment (start 166.1795 97.9805) (end 168.91 95.25) (width 1.25) (layer B.Cu) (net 6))
 (segment (start 157.5435 97.9805) (end 166.1795 97.9805) (width 1.25) (layer B.Cu) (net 6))
 (segment (start 139.7 83.82) (end 138.43 82.55) (width 1.25) (layer B.Cu) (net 7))
 (segment (start 139.7 90.17) (end 139.7 83.82) (width 1.25) (layer B.Cu) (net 7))
 (segment (start 138.43 80.01) (end 140.97 77.47) (width 1.25) (layer B.Cu) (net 7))
 (segment (start 138.43 82.55) (end 138.43 80.01) (width 1.25) (layer B.Cu) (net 7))
 (segment (start 139.7 90.17) (end 143.51 90.17) (width 1.25) (layer B.Cu) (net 7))
 (segment (start 151.13 95.25) (end 151.6507 95.25) (width 1.25) (layer B.Cu) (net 8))
 (segment (start 151.6507 95.25) (end 156.591 100.1903) (width 1.25) (layer B.Cu) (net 8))
 (segment (start 171.8945 91.3765) (end 174.371 88.9) (width 1.25) (layer B.Cu) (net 8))
 (segment (start 163.1315 81.153) (end 160.9344 78.9559) (width 1.25) (layer B.Cu) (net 8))
 (segment (start 157.48 79.7941) (end 157.48 81.28) (width 1.25) (layer B.Cu) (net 8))
 (segment (start 156.591 100.1903) (end 167.6908 100.1903) (width 1.25) (layer B.Cu) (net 8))
 (segment (start 167.6908 100.1903) (end 171.8945 95.9866) (width 1.25) (layer B.Cu) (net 8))
 (segment (start 171.8945 95.9866) (end 171.8945 91.3765) (width 1.25) (layer B.Cu) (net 8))
 (segment (start 174.371 88.9) (end 174.371 84.9503) (width 1.25) (layer B.Cu) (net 8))
 (segment (start 174.371 84.9503) (end 172.1739 82.7532) (width 1.25) (layer B.Cu) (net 8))
 (segment (start 163.2712 82.7532) (end 163.1315 82.6135) (width 1.25) (layer B.Cu) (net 8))
 (segment (start 158.3182 78.9559) (end 157.48 79.7941) (width 1.25) (layer B.Cu) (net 8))
 (segment (start 163.1315 82.6135) (end 163.1315 81.153) (width 1.25) (layer B.Cu) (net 8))
 (segment (start 172.1739 82.7532) (end 163.2712 82.7532) (width 1.25) (layer B.Cu) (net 8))
 (segment (start 160.9344 78.9559) (end 158.3182 78.9559) (width 1.25) (layer B.Cu) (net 8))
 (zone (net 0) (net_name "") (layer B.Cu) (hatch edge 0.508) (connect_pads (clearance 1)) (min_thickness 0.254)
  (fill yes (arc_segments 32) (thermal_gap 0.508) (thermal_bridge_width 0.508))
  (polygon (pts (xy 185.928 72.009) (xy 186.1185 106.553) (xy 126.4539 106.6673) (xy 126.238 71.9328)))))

